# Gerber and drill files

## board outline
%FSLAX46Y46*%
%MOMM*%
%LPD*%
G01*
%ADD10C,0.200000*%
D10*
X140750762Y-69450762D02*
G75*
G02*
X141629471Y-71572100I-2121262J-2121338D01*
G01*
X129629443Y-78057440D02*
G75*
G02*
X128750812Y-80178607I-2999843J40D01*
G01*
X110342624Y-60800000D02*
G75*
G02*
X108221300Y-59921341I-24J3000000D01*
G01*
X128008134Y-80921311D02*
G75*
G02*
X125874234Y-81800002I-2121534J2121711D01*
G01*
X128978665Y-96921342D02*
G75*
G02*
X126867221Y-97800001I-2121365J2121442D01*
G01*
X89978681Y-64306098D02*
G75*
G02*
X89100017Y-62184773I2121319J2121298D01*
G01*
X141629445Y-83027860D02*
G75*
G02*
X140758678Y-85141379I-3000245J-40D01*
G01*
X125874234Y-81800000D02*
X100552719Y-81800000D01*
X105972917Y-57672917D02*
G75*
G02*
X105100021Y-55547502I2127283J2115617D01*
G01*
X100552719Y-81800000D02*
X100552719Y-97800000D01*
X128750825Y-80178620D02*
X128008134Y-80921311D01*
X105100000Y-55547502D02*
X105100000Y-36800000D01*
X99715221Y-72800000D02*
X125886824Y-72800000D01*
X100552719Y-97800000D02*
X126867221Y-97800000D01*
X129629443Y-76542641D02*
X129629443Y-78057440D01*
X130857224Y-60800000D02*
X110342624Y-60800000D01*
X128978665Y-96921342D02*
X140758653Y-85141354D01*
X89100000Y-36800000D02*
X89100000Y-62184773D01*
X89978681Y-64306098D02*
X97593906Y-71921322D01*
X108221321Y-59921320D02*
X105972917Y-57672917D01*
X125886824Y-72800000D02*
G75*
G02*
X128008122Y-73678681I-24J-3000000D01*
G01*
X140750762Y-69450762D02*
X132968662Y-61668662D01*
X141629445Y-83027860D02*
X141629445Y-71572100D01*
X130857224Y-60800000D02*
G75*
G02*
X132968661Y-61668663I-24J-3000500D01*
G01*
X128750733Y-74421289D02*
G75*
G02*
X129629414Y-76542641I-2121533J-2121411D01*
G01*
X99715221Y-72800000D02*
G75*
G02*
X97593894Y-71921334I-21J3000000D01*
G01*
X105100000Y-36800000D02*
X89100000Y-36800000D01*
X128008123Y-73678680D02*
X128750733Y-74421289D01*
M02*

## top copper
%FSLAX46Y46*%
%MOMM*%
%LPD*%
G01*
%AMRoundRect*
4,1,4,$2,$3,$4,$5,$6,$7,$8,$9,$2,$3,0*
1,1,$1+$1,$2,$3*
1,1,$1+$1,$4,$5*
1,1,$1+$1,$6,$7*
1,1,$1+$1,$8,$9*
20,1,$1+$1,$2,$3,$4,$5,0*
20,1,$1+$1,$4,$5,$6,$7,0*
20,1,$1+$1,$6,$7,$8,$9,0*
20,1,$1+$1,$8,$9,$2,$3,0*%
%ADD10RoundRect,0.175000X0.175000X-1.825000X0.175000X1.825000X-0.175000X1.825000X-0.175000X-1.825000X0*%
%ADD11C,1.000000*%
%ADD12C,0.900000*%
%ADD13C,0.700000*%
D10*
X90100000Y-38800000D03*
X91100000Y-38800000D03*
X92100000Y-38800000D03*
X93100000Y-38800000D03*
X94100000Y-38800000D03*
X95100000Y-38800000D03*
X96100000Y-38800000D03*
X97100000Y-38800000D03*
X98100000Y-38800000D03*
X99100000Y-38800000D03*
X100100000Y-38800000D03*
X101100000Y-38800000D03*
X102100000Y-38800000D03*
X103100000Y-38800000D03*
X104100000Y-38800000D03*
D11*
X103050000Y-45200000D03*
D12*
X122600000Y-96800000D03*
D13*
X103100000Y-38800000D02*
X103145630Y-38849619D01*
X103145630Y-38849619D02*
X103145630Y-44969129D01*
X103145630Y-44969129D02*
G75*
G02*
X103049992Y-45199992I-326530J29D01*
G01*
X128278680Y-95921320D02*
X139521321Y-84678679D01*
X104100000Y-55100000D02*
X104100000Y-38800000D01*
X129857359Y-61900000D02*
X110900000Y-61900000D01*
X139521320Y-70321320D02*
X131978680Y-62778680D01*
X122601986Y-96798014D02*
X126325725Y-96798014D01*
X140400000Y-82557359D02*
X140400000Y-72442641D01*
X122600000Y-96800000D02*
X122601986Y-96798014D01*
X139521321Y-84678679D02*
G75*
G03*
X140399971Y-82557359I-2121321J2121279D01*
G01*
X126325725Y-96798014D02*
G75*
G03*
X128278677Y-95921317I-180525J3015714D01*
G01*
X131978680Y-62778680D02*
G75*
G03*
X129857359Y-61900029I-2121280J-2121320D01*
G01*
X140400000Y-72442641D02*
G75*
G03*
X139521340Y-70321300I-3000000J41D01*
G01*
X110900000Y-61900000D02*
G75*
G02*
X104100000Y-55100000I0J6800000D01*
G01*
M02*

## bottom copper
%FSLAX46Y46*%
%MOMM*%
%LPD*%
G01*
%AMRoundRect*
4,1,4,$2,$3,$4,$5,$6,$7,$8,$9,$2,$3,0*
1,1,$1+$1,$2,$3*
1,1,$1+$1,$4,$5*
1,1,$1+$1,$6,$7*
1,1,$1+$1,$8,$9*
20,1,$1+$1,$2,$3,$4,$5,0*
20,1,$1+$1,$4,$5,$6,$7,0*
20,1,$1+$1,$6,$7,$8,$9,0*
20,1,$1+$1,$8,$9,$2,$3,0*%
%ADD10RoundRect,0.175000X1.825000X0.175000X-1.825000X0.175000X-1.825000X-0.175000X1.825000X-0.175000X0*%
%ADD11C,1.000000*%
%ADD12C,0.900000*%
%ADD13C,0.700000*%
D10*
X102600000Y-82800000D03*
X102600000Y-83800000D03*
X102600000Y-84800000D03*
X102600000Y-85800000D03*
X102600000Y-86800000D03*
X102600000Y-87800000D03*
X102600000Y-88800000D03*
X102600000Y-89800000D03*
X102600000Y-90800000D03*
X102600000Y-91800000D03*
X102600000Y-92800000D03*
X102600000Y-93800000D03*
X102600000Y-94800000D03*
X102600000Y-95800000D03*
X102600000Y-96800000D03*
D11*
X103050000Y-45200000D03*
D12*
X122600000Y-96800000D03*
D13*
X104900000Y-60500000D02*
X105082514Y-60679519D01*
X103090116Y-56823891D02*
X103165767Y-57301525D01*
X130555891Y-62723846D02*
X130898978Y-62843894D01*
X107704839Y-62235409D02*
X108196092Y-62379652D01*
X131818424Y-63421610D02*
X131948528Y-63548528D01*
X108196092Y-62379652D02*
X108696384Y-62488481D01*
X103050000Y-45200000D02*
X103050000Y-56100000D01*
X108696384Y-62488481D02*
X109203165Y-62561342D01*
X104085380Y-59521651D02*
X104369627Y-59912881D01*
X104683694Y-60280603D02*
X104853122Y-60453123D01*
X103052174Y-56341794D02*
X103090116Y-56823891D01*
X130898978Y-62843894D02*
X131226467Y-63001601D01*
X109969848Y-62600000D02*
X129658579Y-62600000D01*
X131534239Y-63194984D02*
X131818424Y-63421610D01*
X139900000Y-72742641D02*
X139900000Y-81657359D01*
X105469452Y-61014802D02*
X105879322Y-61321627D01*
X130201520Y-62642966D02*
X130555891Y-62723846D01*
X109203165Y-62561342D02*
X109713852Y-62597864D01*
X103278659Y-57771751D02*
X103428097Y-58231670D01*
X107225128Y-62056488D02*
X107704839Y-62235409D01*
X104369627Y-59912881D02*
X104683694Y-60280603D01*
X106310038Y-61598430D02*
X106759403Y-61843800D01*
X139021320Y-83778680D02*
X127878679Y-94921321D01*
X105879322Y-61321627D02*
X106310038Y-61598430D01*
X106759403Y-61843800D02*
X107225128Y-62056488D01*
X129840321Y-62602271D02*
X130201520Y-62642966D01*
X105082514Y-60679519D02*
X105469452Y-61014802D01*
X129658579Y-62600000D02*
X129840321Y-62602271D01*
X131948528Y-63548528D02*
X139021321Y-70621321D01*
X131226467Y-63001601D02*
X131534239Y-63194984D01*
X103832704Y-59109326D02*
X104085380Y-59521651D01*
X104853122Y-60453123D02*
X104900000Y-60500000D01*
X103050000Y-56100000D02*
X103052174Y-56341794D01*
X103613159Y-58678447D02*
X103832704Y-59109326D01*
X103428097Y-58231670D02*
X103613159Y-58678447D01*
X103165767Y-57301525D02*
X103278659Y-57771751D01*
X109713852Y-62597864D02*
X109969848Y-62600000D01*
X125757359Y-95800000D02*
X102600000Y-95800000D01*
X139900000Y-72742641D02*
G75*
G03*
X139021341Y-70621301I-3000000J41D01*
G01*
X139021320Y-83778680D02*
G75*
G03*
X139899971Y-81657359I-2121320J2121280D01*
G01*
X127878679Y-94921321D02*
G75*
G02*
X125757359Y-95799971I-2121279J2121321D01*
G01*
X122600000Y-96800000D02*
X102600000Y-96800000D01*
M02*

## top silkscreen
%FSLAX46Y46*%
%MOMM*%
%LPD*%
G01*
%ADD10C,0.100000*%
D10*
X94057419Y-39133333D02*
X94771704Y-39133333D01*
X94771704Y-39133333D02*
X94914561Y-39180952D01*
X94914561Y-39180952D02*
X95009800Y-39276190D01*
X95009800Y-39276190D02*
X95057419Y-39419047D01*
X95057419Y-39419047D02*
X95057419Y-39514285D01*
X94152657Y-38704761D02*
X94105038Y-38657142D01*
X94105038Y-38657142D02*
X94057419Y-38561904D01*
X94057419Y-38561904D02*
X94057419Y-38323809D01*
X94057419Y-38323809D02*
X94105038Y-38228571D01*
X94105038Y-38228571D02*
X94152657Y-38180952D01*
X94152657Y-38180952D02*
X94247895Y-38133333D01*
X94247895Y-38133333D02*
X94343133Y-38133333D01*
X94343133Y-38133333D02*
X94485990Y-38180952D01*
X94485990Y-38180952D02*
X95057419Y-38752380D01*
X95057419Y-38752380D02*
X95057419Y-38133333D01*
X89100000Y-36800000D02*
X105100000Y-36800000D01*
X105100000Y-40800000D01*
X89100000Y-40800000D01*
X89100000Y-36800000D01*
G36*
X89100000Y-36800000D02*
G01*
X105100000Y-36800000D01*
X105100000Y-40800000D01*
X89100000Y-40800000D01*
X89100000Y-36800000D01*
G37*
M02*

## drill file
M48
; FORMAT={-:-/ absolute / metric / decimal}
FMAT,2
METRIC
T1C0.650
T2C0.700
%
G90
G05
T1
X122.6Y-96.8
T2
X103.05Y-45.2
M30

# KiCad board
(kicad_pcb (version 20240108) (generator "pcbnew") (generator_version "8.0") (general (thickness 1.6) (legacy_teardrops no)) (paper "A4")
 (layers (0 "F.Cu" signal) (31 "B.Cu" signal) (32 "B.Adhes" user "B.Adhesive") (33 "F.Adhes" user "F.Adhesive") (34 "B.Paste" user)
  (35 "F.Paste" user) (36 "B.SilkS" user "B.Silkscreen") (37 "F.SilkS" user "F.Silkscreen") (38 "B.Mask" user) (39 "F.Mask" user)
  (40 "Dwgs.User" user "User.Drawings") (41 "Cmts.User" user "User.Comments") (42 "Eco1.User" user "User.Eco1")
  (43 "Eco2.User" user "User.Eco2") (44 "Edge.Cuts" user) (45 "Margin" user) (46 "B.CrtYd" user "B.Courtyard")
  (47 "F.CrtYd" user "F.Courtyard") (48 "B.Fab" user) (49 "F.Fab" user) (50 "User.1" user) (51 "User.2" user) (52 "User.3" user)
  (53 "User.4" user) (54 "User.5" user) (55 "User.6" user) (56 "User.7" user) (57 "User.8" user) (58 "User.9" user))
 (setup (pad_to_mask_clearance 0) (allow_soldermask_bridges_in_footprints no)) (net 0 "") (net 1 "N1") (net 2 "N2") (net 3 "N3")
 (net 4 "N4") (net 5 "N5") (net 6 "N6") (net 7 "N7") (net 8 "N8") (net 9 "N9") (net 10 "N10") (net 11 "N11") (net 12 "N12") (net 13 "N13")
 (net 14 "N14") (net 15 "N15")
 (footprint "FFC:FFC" (layer "F.Cu") (at 97.1 38.8 90)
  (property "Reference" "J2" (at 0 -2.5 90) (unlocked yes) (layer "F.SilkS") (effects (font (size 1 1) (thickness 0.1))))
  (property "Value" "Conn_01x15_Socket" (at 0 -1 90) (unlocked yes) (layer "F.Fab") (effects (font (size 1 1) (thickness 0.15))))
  (fp_rect (start -2 -8) (end 2 8) (stroke (width 0.1) (type solid)) (fill solid) (layer "F.SilkS"))
  (pad "1" smd roundrect (at 0 -7 90) (size 4 0.7) (layers "F.Cu" "F.Paste" "F.Mask") (roundrect_rratio 0.25) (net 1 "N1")
   (thermal_bridge_angle 45))
  (pad "2" smd roundrect (at 0 -6 90) (size 4 0.7) (layers "F.Cu" "F.Paste" "F.Mask") (roundrect_rratio 0.25) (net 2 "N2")
   (thermal_bridge_angle 45))
  (pad "3" smd roundrect (at 0 -5 90) (size 4 0.7) (layers "F.Cu" "F.Paste" "F.Mask") (roundrect_rratio 0.25) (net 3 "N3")
   (thermal_bridge_angle 45))
  (pad "4" smd roundrect (at 0 -4 90) (size 4 0.7) (layers "F.Cu" "F.Paste" "F.Mask") (roundrect_rratio 0.25) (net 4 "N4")
   (thermal_bridge_angle 45))
  (pad "5" smd roundrect (at 0 -3 90) (size 4 0.7) (layers "F.Cu" "F.Paste" "F.Mask") (roundrect_rratio 0.25) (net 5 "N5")
   (thermal_bridge_angle 45))
  (pad "6" smd roundrect (at 0 -2 90) (size 4 0.7) (layers "F.Cu" "F.Paste" "F.Mask") (roundrect_rratio 0.25) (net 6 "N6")
   (thermal_bridge_angle 45))
  (pad "7" smd roundrect (at 0 -1 90) (size 4 0.7) (layers "F.Cu" "F.Paste" "F.Mask") (roundrect_rratio 0.25) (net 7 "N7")
   (thermal_bridge_angle 45))
  (pad "8" smd roundrect (at 0 0 90) (size 4 0.7) (layers "F.Cu" "F.Paste" "F.Mask") (roundrect_rratio 0.25) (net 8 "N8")
   (thermal_bridge_angle 45))
  (pad "9" smd roundrect (at 0 1 90) (size 4 0.7) (layers "F.Cu" "F.Paste" "F.Mask") (roundrect_rratio 0.25) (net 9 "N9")
   (thermal_bridge_angle 45))
  (pad "10" smd roundrect (at 0 2 90) (size 4 0.7) (layers "F.Cu" "F.Paste" "F.Mask") (roundrect_rratio 0.25) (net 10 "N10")
   (thermal_bridge_angle 45))
  (pad "11" smd roundrect (at 0 3 90) (size 4 0.7) (layers "F.Cu" "F.Paste" "F.Mask") (roundrect_rratio 0.25) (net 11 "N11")
   (thermal_bridge_angle 45))
  (pad "12" smd roundrect (at 0 4 90) (size 4 0.7) (layers "F.Cu" "F.Paste" "F.Mask") (roundrect_rratio 0.25) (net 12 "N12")
   (thermal_bridge_angle 45))
  (pad "13" smd roundrect (at 0 5 90) (size 4 0.7) (layers "F.Cu" "F.Paste" "F.Mask") (roundrect_rratio 0.25) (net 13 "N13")
   (thermal_bridge_angle 45))
  (pad "14" smd roundrect (at 0 6 90) (size 4 0.7) (layers "F.Cu" "F.Paste" "F.Mask") (roundrect_rratio 0.25) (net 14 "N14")
   (thermal_bridge_angle 45))
  (pad "15" smd roundrect (at 0 7 90) (size 4 0.7) (layers "F.Cu" "F.Paste" "F.Mask") (roundrect_rratio 0.25) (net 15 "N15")
   (thermal_bridge_angle 45)))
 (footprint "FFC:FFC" (layer "B.Cu") (at 102.6 89.8 180)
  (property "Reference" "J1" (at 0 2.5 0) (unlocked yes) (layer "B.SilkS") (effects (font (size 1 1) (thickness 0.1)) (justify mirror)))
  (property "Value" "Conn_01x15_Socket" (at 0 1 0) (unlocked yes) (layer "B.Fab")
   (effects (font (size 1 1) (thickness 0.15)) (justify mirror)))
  (pad "1" smd roundrect (at 0 7 180) (size 4 0.7) (layers "B.Cu" "B.Paste" "B.Mask") (roundrect_rratio 0.25) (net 1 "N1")
   (thermal_bridge_angle 45))
  (pad "2" smd roundrect (at 0 6 180) (size 4 0.7) (layers "B.Cu" "B.Paste" "B.Mask") (roundrect_rratio 0.25) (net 2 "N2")
   (thermal_bridge_angle 45))
  (pad "3" smd roundrect (at 0 5 180) (size 4 0.7) (layers "B.Cu" "B.Paste" "B.Mask") (roundrect_rratio 0.25) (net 3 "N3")
   (thermal_bridge_angle 45))
  (pad "4" smd roundrect (at 0 4 180) (size 4 0.7) (layers "B.Cu" "B.Paste" "B.Mask") (roundrect_rratio 0.25) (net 4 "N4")
   (thermal_bridge_angle 45))
  (pad "5" smd roundrect (at 0 3 180) (size 4 0.7) (layers "B.Cu" "B.Paste" "B.Mask") (roundrect_rratio 0.25) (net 5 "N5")
   (thermal_bridge_angle 45))
  (pad "6" smd roundrect (at 0 2 180) (size 4 0.7) (layers "B.Cu" "B.Paste" "B.Mask") (roundrect_rratio 0.25) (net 6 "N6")
   (thermal_bridge_angle 45))
  (pad "7" smd roundrect (at 0 1 180) (size 4 0.7) (layers "B.Cu" "B.Paste" "B.Mask") (roundrect_rratio 0.25) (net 7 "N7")
   (thermal_bridge_angle 45))
  (pad "8" smd roundrect (at 0 0 180) (size 4 0.7) (layers "B.Cu" "B.Paste" "B.Mask") (roundrect_rratio 0.25) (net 8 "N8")
   (thermal_bridge_angle 45))
  (pad "9" smd roundrect (at 0 -1 180) (size 4 0.7) (layers "B.Cu" "B.Paste" "B.Mask") (roundrect_rratio 0.25) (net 9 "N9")
   (thermal_bridge_angle 45))
  (pad "10" smd roundrect (at 0 -2 180) (size 4 0.7) (layers "B.Cu" "B.Paste" "B.Mask") (roundrect_rratio 0.25) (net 10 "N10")
   (thermal_bridge_angle 45))
  (pad "11" smd roundrect (at 0 -3 180) (size 4 0.7) (layers "B.Cu" "B.Paste" "B.Mask") (roundrect_rratio 0.25) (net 11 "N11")
   (thermal_bridge_angle 45))
  (pad "12" smd roundrect (at 0 -4 180) (size 4 0.7) (layers "B.Cu" "B.Paste" "B.Mask") (roundrect_rratio 0.25) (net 12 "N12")
   (thermal_bridge_angle 45))
  (pad "13" smd roundrect (at 0 -5 180) (size 4 0.7) (layers "B.Cu" "B.Paste" "B.Mask") (roundrect_rratio 0.25) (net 13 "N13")
   (thermal_bridge_angle 45))
  (pad "14" smd roundrect (at 0 -6 180) (size 4 0.7) (layers "B.Cu" "B.Paste" "B.Mask") (roundrect_rratio 0.25) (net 14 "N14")
   (thermal_bridge_angle 45))
  (pad "15" smd roundrect (at 0 -7 180) (size 4 0.7) (layers "B.Cu" "B.Paste" "B.Mask") (roundrect_rratio 0.25) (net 15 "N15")
   (thermal_bridge_angle 45)))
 (gr_arc (start 140.750762 69.450762) (mid 141.401086 70.42404) (end 141.629445 71.5721) (stroke (width 0.2) (type default))
  (layer "Edge.Cuts"))
 (gr_arc (start 129.629443 78.05744) (mid 129.401097 79.205413) (end 128.750825 80.17862) (stroke (width 0.2) (type default))
  (layer "Edge.Cuts"))
 (gr_arc (start 110.342624 60.8) (mid 109.194585 60.571635) (end 108.221321 59.92132) (stroke (width 0.2) (type default))
  (layer "Edge.Cuts"))
 (gr_arc (start 128.008134 80.921311) (mid 127.029045 81.574019) (end 125.874234 81.8) (stroke (width 0.2) (type default))
  (layer "Edge.Cuts"))
 (gr_arc (start 128.978665 96.921342) (mid 128.009955 97.569757) (end 126.867221 97.8) (stroke (width 0.2) (type default))
  (layer "Edge.Cuts"))
 (gr_arc (start 89.978681 64.306098) (mid 89.328361 63.332826) (end 89.1 62.184773) (stroke (width 0.2) (type default)) (layer "Edge.Cuts"))
 (gr_arc (start 141.629445 83.02786) (mid 141.403217 84.170787) (end 140.758653 85.141354) (stroke (width 0.2) (type default))
  (layer "Edge.Cuts"))
 (gr_line (start 125.874234 81.8) (end 100.552719 81.8) (stroke (width 0.2) (type default)) (layer "Edge.Cuts"))
 (gr_arc (start 105.972917 57.672917) (mid 105.324931 56.697085) (end 105.1 55.547502) (stroke (width 0.2) (type default))
  (layer "Edge.Cuts"))
 (gr_line (start 100.552719 81.8) (end 100.552719 97.8) (stroke (width 0.2) (type default)) (layer "Edge.Cuts"))
 (gr_line (start 128.750825 80.17862) (end 128.008134 80.921311) (stroke (width 0.2) (type default)) (layer "Edge.Cuts"))
 (gr_line (start 105.1 55.547502) (end 105.1 36.8) (stroke (width 0.2) (type default)) (layer "Edge.Cuts"))
 (gr_line (start 99.715221 72.8) (end 125.886824 72.8) (stroke (width 0.2) (type default)) (layer "Edge.Cuts"))
 (gr_line (start 100.552719 97.8) (end 126.867221 97.8) (stroke (width 0.2) (type default)) (layer "Edge.Cuts"))
 (gr_line (start 129.629443 76.542641) (end 129.629443 78.05744) (stroke (width 0.2) (type default)) (layer "Edge.Cuts"))
 (gr_line (start 130.857224 60.8) (end 110.342624 60.8) (stroke (width 0.2) (type default)) (layer "Edge.Cuts"))
 (gr_line (start 128.978665 96.921342) (end 140.758653 85.141354) (stroke (width 0.2) (type default)) (layer "Edge.Cuts"))
 (gr_line (start 89.1 36.8) (end 89.1 62.184773) (stroke (width 0.2) (type default)) (layer "Edge.Cuts"))
 (gr_line (start 89.978681 64.306098) (end 97.593906 71.921322) (stroke (width 0.2) (type default)) (layer "Edge.Cuts"))
 (gr_line (start 108.221321 59.92132) (end 105.972917 57.672917) (stroke (width 0.2) (type default)) (layer "Edge.Cuts"))
 (gr_arc (start 125.886824 72.8) (mid 127.034862 73.028364) (end 128.008123 73.67868) (stroke (width 0.2) (type default))
  (layer "Edge.Cuts"))
 (gr_line (start 140.750762 69.450762) (end 132.968662 61.668662) (stroke (width 0.2) (type default)) (layer "Edge.Cuts"))
 (gr_line (start 141.629445 83.02786) (end 141.629445 71.5721) (stroke (width 0.2) (type default)) (layer "Edge.Cuts"))
 (gr_arc (start 130.857224 60.8) (mid 131.998793 61.025653) (end 132.968662 61.668662) (stroke (width 0.2) (type default))
  (layer "Edge.Cuts"))
 (gr_arc (start 128.750733 74.421289) (mid 129.401057 75.394574) (end 129.629443 76.542641) (stroke (width 0.2) (type default))
  (layer "Edge.Cuts"))
 (gr_arc (start 99.715221 72.8) (mid 98.567174 72.571639) (end 97.593906 71.921322) (stroke (width 0.2) (type default)) (layer "Edge.Cuts"))
 (gr_line (start 105.1 36.8) (end 89.1 36.8) (stroke (width 0.2) (type default)) (layer "Edge.Cuts"))
 (gr_line (start 128.008123 73.67868) (end 128.750733 74.421289) (stroke (width 0.2) (type default)) (layer "Edge.Cuts"))
 (segment (start 103.1 38.8) (end 103.14563 38.849619) (width 0.7) (layer "F.Cu") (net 14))
 (segment (start 103.14563 38.849619) (end 103.14563 44.969129) (width 0.7) (layer "F.Cu") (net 14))
 (via (at 103.05 45.2) (size 1) (drill 0.7) (layers "F.Cu" "B.Cu") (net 14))
 (arc (start 103.14563 44.969129) (mid 103.120776 45.094075) (end 103.05 45.2) (width 0.7) (layer "F.Cu") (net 14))
 (segment (start 104.9 60.5) (end 105.082514 60.679519) (width 0.7) (layer "B.Cu") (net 14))
 (segment (start 103.090116 56.823891) (end 103.165767 57.301525) (width 0.7) (layer "B.Cu") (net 14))
 (segment (start 130.555891 62.723846) (end 130.898978 62.843894) (width 0.7) (layer "B.Cu") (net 14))
 (segment (start 107.704839 62.235409) (end 108.196092 62.379652) (width 0.7) (layer "B.Cu") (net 14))
 (segment (start 131.818424 63.42161) (end 131.948528 63.548528) (width 0.7) (layer "B.Cu") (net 14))
 (segment (start 108.196092 62.379652) (end 108.696384 62.488481) (width 0.7) (layer "B.Cu") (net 14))
 (segment (start 103.05 45.2) (end 103.05 56.1) (width 0.7) (layer "B.Cu") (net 14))
 (segment (start 108.696384 62.488481) (end 109.203165 62.561342) (width 0.7) (layer "B.Cu") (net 14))
 (segment (start 104.08538 59.521651) (end 104.369627 59.912881) (width 0.7) (layer "B.Cu") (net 14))
 (segment (start 104.683694 60.280603) (end 104.853122 60.453123) (width 0.7) (layer "B.Cu") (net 14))
 (segment (start 103.052174 56.341794) (end 103.090116 56.823891) (width 0.7) (layer "B.Cu") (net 14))
 (segment (start 130.898978 62.843894) (end 131.226467 63.001601) (width 0.7) (layer "B.Cu") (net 14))
 (segment (start 109.969848 62.6) (end 129.658579 62.6) (width 0.7) (layer "B.Cu") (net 14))
 (segment (start 131.534239 63.194984) (end 131.818424 63.42161) (width 0.7) (layer "B.Cu") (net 14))
 (segment (start 139.9 72.742641) (end 139.9 81.657359) (width 0.7) (layer "B.Cu") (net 14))
 (segment (start 105.469452 61.014802) (end 105.879322 61.321627) (width 0.7) (layer "B.Cu") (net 14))
 (segment (start 130.20152 62.642966) (end 130.555891 62.723846) (width 0.7) (layer "B.Cu") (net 14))
 (segment (start 109.203165 62.561342) (end 109.713852 62.597864) (width 0.7) (layer "B.Cu") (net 14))
 (segment (start 103.278659 57.771751) (end 103.428097 58.23167) (width 0.7) (layer "B.Cu") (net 14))
 (segment (start 107.225128 62.056488) (end 107.704839 62.235409) (width 0.7) (layer "B.Cu") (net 14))
 (segment (start 104.369627 59.912881) (end 104.683694 60.280603) (width 0.7) (layer "B.Cu") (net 14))
 (segment (start 106.310038 61.59843) (end 106.759403 61.8438) (width 0.7) (layer "B.Cu") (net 14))
 (segment (start 139.02132 83.77868) (end 127.878679 94.921321) (width 0.7) (layer "B.Cu") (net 14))
 (segment (start 105.879322 61.321627) (end 106.310038 61.59843) (width 0.7) (layer "B.Cu") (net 14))
 (segment (start 106.759403 61.8438) (end 107.225128 62.056488) (width 0.7) (layer "B.Cu") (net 14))
 (segment (start 129.840321 62.602271) (end 130.20152 62.642966) (width 0.7) (layer "B.Cu") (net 14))
 (segment (start 105.082514 60.679519) (end 105.469452 61.014802) (width 0.7) (layer "B.Cu") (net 14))
 (segment (start 129.658579 62.6) (end 129.840321 62.602271) (width 0.7) (layer "B.Cu") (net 14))
 (segment (start 131.948528 63.548528) (end 139.021321 70.621321) (width 0.7) (layer "B.Cu") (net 14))
 (segment (start 131.226467 63.001601) (end 131.534239 63.194984) (width 0.7) (layer "B.Cu") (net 14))
 (segment (start 103.832704 59.109326) (end 104.08538 59.521651) (width 0.7) (layer "B.Cu") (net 14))
 (segment (start 104.853122 60.453123) (end 104.9 60.5) (width 0.7) (layer "B.Cu") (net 14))
 (segment (start 103.05 56.1) (end 103.052174 56.341794) (width 0.7) (layer "B.Cu") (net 14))
 (segment (start 103.613159 58.678447) (end 103.832704 59.109326) (width 0.7) (layer "B.Cu") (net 14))
 (segment (start 103.428097 58.23167) (end 103.613159 58.678447) (width 0.7) (layer "B.Cu") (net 14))
 (segment (start 103.165767 57.301525) (end 103.278659 57.771751) (width 0.7) (layer "B.Cu") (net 14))
 (segment (start 109.713852 62.597864) (end 109.969848 62.6) (width 0.7) (layer "B.Cu") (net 14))
 (segment (start 125.757359 95.8) (end 102.6 95.8) (width 0.7) (layer "B.Cu") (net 14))
 (arc (start 139.9 72.742641) (mid 139.671639 71.594591) (end 139.021321 70.621321) (width 0.7) (layer "B.Cu") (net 14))
 (arc (start 139.02132 83.77868) (mid 139.671639 82.80541) (end 139.9 81.657359) (width 0.7) (layer "B.Cu") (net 14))
 (arc (start 127.878679 94.921321) (mid 126.905409 95.571639) (end 125.757359 95.8) (width 0.7) (layer "B.Cu") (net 14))
 (segment (start 128.27868 95.92132) (end 139.521321 84.678679) (width 0.7) (layer "F.Cu") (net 15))
 (segment (start 104.1 55.1) (end 104.1 38.8) (width 0.7) (layer "F.Cu") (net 15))
 (segment (start 129.857359 61.9) (end 110.9 61.9) (width 0.7) (layer "F.Cu") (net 15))
 (segment (start 139.52132 70.32132) (end 131.97868 62.77868) (width 0.7) (layer "F.Cu") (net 15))
 (segment (start 122.601986 96.798014) (end 126.325725 96.798014) (width 0.7) (layer "F.Cu") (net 15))
 (segment (start 140.4 82.557359) (end 140.4 72.442641) (width 0.7) (layer "F.Cu") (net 15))
 (segment (start 122.6 96.8) (end 122.601986 96.798014) (width 0.7) (layer "F.Cu") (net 15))
 (via (at 122.6 96.8) (size 0.9) (drill 0.65) (layers "F.Cu" "B.Cu") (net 15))
 (arc (start 139.521321 84.678679) (mid 140.171639 83.705409) (end 140.4 82.557359) (width 0.7) (layer "F.Cu") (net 15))
 (arc (start 126.325725 96.798014) (mid 127.38269 96.538337) (end 128.27868 95.92132) (width 0.7) (layer "F.Cu") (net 15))
 (arc (start 131.97868 62.77868) (mid 131.00541 62.128361) (end 129.857359 61.9) (width 0.7) (layer "F.Cu") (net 15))
 (arc (start 140.4 72.442641) (mid 140.171638 71.29459) (end 139.52132 70.32132) (width 0.7) (layer "F.Cu") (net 15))
 (arc (start 110.9 61.9) (mid 106.091674 59.908326) (end 104.1 55.1) (width 0.7) (layer "F.Cu") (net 15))
 (segment (start 122.6 96.8) (end 102.6 96.8) (width 0.7) (layer "B.Cu") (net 15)))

